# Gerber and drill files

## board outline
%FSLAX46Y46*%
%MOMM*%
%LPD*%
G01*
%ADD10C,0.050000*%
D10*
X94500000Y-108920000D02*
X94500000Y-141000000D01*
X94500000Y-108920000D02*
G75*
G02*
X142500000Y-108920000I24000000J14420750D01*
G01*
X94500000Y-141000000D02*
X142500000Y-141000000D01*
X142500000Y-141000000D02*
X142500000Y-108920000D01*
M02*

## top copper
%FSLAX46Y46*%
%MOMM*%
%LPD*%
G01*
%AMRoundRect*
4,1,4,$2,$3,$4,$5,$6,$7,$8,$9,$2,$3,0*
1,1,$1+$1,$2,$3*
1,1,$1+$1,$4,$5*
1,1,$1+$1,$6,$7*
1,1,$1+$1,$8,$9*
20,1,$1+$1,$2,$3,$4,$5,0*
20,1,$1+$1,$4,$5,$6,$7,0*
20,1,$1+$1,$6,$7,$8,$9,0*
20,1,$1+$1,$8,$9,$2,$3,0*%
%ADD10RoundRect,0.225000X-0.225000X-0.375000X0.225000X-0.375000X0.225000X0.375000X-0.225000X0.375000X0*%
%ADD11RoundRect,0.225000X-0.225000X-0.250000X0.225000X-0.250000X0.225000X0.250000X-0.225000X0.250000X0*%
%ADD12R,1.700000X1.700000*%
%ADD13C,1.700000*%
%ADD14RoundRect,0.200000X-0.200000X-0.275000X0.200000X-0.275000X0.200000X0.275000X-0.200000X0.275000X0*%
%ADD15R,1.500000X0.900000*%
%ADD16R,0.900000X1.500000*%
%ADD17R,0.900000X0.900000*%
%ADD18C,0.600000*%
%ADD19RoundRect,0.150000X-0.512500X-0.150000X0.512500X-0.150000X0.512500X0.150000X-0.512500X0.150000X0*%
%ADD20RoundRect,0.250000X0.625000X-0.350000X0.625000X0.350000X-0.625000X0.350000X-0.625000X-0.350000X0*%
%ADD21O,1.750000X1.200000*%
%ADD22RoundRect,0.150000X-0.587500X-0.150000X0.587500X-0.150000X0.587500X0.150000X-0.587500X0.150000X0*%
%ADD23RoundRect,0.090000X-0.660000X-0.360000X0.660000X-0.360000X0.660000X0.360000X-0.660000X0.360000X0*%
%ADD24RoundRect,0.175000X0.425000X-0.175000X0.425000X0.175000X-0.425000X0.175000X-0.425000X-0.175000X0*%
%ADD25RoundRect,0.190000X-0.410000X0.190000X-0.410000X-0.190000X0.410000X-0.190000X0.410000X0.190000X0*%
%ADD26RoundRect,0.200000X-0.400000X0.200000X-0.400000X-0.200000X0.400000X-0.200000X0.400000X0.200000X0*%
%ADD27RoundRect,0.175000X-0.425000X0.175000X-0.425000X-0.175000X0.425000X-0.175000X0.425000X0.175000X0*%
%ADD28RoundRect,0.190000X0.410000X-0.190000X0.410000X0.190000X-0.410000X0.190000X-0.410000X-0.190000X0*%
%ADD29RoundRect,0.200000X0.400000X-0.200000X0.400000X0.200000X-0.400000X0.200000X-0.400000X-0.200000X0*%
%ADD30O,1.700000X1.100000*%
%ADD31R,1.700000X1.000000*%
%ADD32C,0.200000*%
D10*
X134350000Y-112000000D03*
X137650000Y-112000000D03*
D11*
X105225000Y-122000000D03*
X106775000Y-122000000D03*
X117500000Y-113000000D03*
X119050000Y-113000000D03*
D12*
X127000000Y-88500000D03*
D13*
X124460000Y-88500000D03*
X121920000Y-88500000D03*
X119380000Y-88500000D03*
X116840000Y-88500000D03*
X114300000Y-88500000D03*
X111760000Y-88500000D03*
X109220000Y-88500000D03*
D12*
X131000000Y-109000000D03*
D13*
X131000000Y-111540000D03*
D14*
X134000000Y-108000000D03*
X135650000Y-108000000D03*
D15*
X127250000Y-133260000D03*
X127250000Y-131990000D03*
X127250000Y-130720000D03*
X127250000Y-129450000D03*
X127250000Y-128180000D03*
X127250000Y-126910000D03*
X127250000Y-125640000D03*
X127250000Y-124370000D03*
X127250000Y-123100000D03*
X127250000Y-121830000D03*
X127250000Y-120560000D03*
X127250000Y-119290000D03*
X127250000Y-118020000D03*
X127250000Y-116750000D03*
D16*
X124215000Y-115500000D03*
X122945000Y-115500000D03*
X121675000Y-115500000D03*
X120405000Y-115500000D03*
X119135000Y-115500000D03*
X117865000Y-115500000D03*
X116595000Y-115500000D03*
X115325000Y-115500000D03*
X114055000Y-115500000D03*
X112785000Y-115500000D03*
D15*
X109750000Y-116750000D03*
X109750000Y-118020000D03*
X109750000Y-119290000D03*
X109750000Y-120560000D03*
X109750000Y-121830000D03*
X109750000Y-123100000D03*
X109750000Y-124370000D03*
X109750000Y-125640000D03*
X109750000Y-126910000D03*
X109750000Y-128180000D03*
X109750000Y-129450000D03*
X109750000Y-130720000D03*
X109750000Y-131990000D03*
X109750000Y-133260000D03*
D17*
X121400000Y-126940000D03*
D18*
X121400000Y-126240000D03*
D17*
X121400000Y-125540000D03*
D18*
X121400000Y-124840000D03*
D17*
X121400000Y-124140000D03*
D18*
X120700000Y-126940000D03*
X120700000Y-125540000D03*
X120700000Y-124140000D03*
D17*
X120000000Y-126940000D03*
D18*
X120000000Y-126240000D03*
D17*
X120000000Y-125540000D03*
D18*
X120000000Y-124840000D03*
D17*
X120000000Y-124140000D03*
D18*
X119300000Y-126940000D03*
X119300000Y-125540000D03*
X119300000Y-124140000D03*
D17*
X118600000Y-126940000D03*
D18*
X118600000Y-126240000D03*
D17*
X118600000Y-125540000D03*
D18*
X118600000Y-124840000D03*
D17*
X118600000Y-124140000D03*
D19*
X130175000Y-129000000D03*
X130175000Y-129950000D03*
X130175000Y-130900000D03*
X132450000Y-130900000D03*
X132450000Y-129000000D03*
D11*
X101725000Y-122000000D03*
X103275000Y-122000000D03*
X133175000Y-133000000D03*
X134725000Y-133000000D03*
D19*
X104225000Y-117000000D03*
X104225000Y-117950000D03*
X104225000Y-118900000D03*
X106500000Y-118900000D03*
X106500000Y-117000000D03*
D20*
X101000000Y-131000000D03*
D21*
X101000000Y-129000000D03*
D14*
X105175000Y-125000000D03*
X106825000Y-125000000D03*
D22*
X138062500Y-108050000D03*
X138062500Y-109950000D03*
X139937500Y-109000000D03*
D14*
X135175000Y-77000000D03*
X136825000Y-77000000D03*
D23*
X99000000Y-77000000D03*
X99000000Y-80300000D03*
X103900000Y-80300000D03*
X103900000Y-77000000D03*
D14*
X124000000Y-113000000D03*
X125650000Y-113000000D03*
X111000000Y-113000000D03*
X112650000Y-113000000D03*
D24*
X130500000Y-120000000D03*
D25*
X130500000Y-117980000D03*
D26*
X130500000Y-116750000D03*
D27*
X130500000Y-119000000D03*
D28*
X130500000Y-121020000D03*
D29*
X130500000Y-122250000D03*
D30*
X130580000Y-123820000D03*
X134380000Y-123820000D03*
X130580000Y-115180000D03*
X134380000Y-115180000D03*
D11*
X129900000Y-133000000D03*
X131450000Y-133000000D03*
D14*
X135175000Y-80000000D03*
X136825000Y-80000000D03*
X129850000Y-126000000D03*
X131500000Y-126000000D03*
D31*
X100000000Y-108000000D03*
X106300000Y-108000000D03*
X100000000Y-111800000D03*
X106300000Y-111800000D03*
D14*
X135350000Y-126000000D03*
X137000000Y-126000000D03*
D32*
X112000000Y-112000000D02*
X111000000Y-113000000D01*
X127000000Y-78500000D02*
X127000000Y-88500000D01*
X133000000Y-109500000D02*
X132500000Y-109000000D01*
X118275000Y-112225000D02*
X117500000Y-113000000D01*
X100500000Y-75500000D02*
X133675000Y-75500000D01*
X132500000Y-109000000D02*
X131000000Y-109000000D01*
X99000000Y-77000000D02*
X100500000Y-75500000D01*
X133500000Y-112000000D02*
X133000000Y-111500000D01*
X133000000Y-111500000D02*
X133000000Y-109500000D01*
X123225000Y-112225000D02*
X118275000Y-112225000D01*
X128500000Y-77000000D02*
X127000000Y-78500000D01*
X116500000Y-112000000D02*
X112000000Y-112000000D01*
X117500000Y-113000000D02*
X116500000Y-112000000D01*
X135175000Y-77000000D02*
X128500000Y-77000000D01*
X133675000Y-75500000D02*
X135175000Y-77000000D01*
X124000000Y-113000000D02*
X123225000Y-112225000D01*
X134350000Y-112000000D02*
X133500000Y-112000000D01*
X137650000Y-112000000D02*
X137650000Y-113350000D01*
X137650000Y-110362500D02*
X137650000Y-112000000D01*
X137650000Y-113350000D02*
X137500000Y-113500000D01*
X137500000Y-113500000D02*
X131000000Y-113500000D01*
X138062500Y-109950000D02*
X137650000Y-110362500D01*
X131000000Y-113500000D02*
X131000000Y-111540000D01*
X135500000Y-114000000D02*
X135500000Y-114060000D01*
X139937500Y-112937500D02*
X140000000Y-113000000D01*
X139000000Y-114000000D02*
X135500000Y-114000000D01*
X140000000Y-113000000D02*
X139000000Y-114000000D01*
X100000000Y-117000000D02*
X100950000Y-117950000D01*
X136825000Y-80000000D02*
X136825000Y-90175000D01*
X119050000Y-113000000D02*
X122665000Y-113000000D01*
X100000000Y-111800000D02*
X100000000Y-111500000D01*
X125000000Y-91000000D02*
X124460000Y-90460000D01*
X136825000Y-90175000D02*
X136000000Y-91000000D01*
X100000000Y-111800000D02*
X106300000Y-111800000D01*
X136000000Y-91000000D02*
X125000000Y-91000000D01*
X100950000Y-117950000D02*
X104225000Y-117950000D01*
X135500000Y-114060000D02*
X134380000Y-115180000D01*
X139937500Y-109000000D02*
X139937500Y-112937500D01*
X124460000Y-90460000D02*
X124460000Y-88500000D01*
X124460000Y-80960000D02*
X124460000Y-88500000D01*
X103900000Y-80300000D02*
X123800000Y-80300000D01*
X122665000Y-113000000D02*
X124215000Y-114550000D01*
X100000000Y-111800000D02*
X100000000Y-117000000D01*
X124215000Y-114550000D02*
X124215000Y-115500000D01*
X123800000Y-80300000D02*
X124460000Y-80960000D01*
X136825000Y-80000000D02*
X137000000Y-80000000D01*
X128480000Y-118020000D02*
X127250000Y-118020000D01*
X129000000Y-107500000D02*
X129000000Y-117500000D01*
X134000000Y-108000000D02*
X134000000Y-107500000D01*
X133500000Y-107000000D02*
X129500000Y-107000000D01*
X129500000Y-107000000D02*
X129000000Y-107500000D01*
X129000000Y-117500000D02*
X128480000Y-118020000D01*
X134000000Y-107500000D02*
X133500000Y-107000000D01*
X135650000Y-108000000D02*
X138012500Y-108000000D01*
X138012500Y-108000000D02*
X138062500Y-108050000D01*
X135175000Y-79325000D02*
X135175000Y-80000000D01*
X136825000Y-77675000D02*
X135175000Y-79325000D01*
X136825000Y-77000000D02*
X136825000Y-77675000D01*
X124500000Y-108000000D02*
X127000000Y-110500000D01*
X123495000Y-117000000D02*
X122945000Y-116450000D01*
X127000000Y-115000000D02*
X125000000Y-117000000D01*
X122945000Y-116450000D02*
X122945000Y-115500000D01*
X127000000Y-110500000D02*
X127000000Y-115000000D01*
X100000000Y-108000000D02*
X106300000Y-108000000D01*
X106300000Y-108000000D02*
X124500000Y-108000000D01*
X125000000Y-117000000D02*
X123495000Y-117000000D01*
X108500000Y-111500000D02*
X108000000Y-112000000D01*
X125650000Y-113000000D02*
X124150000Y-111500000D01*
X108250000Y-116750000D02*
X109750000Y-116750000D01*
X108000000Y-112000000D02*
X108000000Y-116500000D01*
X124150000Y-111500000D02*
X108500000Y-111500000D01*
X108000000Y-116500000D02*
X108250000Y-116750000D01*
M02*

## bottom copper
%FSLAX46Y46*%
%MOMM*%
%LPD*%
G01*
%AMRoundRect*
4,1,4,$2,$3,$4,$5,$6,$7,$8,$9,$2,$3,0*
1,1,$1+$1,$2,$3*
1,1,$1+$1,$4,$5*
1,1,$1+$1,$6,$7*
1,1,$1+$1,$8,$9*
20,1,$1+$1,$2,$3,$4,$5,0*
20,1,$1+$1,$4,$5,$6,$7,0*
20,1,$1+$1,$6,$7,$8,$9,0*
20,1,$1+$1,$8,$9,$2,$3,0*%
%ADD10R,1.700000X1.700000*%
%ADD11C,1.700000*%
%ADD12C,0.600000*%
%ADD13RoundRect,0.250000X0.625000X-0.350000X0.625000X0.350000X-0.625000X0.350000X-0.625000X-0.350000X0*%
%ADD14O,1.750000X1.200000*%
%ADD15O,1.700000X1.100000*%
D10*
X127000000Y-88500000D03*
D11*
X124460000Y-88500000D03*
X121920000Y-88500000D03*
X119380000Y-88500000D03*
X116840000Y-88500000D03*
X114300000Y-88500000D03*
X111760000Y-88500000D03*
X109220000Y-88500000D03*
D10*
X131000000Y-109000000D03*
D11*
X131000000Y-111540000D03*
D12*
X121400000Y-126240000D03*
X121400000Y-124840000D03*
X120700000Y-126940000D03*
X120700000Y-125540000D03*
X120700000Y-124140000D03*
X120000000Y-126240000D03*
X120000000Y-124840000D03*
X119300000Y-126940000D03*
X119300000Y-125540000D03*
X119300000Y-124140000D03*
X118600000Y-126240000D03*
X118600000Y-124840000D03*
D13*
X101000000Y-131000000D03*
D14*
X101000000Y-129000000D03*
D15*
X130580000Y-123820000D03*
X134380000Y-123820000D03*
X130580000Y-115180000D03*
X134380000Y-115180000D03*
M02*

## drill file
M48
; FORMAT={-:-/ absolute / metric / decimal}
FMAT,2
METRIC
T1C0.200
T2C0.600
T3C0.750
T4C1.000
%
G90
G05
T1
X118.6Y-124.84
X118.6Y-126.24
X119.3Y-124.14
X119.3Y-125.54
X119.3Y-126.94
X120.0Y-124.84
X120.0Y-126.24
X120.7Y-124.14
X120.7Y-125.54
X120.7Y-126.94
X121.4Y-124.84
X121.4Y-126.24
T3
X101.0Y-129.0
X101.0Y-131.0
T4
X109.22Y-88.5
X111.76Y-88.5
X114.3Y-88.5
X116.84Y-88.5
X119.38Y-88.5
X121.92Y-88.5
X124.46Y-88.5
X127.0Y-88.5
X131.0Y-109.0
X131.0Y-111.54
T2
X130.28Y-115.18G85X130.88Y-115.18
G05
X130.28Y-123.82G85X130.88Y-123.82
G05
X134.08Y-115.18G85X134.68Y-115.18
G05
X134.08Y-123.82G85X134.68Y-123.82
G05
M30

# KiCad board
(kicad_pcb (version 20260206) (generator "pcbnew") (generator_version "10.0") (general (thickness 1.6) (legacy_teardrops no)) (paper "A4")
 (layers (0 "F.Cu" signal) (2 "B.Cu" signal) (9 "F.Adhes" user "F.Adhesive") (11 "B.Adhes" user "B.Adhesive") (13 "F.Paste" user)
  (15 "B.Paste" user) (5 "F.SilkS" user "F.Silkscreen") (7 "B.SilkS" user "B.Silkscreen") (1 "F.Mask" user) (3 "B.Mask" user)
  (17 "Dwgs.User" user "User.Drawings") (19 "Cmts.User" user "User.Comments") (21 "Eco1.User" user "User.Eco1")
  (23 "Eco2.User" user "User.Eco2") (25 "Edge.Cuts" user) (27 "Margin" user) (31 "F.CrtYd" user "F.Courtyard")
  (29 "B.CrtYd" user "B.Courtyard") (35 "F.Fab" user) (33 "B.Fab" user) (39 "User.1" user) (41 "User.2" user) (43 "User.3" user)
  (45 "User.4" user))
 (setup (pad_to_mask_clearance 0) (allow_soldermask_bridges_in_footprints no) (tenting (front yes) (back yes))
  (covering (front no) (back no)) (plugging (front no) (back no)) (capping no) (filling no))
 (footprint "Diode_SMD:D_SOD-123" (layer "F.Cu") (at 136 112)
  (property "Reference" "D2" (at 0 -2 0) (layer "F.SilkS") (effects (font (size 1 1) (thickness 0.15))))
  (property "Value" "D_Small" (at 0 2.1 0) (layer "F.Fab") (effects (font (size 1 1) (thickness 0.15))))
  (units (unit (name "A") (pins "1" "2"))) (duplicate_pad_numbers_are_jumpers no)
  (pad "1" smd roundrect (at -1.65 0) (size 0.9 1.2) (layers "F.Cu" "F.Mask" "F.Paste") (roundrect_rratio 0.25) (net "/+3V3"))
  (pad "2" smd roundrect (at 1.65 0) (size 0.9 1.2) (layers "F.Cu" "F.Mask" "F.Paste") (roundrect_rratio 0.25) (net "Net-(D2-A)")))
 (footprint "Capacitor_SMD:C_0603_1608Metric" (layer "F.Cu") (at 106 122)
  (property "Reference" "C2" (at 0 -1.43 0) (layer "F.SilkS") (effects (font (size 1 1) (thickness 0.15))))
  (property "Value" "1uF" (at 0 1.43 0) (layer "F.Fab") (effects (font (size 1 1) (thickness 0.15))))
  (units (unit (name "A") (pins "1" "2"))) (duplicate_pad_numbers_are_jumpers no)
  (pad "1" smd roundrect (at -0.775 0) (size 0.9 0.95) (layers "F.Cu" "F.Mask" "F.Paste") (roundrect_rratio 0.25) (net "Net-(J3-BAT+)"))
  (pad "2" smd roundrect (at 0.775 0) (size 0.9 0.95) (layers "F.Cu" "F.Mask" "F.Paste") (roundrect_rratio 0.25) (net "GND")))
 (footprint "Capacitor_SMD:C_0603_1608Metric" (layer "F.Cu") (at 118.275 113)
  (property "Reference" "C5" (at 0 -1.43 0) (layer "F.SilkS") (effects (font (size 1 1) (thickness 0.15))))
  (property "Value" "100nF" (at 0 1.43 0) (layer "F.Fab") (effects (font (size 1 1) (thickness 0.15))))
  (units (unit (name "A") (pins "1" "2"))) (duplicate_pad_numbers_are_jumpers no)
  (pad "1" smd roundrect (at -0.775 0) (size 0.9 0.95) (layers "F.Cu" "F.Mask" "F.Paste") (roundrect_rratio 0.25) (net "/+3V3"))
  (pad "2" smd roundrect (at 0.775 0) (size 0.9 0.95) (layers "F.Cu" "F.Mask" "F.Paste") (roundrect_rratio 0.25) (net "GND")))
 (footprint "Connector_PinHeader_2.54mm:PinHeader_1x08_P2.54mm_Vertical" (layer "F.Cu") (at 127 88.5 -90)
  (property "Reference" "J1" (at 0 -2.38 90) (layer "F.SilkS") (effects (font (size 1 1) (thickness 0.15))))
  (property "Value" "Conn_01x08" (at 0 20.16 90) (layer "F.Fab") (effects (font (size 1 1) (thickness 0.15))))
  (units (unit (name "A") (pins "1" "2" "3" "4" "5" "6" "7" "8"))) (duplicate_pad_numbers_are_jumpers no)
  (pad "1" thru_hole rect (at 0 0 270) (size 1.7 1.7) (drill 1) (layers "*.Cu" "*.Mask") (remove_unused_layers no) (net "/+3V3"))
  (pad "2" thru_hole circle (at 0 2.54 270) (size 1.7 1.7) (drill 1) (layers "*.Cu" "*.Mask") (remove_unused_layers no) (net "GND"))
  (pad "3" thru_hole circle (at 0 5.08 270) (size 1.7 1.7) (drill 1) (layers "*.Cu" "*.Mask") (remove_unused_layers no) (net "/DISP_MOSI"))
  (pad "4" thru_hole circle (at 0 7.62 270) (size 1.7 1.7) (drill 1) (layers "*.Cu" "*.Mask") (remove_unused_layers no) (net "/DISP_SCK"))
  (pad "5" thru_hole circle (at 0 10.16 270) (size 1.7 1.7) (drill 1) (layers "*.Cu" "*.Mask") (remove_unused_layers no) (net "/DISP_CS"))
  (pad "6" thru_hole circle (at 0 12.7 270) (size 1.7 1.7) (drill 1) (layers "*.Cu" "*.Mask") (remove_unused_layers no) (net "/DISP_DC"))
  (pad "7" thru_hole circle (at 0 15.24 270) (size 1.7 1.7) (drill 1) (layers "*.Cu" "*.Mask") (remove_unused_layers no) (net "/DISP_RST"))
  (pad "8" thru_hole circle (at 0 17.78 270) (size 1.7 1.7) (drill 1) (layers "*.Cu" "*.Mask") (remove_unused_layers no) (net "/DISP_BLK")))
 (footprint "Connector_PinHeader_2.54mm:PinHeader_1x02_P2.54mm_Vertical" (layer "F.Cu") (at 131 109)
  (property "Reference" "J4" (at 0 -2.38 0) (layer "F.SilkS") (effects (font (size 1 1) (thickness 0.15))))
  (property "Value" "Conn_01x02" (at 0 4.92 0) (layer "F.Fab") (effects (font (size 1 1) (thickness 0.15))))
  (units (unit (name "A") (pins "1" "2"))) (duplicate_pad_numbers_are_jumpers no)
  (pad "1" thru_hole rect (at 0 0) (size 1.7 1.7) (drill 1) (layers "*.Cu" "*.Mask") (remove_unused_layers no) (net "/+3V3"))
  (pad "2" thru_hole circle (at 0 2.54) (size 1.7 1.7) (drill 1) (layers "*.Cu" "*.Mask") (remove_unused_layers no) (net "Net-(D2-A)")))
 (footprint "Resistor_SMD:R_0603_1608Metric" (layer "F.Cu") (at 134.825 108)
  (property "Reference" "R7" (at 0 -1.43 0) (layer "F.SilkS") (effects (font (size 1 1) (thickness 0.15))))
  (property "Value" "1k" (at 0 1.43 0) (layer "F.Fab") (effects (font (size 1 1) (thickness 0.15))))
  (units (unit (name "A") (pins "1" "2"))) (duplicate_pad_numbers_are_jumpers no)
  (pad "1" smd roundrect (at -0.825 0) (size 0.8 0.95) (layers "F.Cu" "F.Mask" "F.Paste") (roundrect_rratio 0.25) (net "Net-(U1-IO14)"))
  (pad "2" smd roundrect (at 0.825 0) (size 0.8 0.95) (layers "F.Cu" "F.Mask" "F.Paste") (roundrect_rratio 0.25) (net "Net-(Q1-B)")))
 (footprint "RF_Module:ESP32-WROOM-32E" (layer "F.Cu") (at 118.5 128 180)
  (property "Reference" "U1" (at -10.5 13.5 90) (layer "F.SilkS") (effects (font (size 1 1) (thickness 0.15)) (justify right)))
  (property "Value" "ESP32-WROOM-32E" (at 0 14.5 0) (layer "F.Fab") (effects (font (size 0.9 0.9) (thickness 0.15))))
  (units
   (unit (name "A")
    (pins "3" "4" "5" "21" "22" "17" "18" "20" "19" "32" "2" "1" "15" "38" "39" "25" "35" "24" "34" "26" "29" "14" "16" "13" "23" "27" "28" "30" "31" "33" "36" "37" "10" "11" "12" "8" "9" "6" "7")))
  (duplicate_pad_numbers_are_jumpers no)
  (pad "1" smd rect (at -8.75 -5.26 180) (size 1.5 0.9) (layers "F.Cu" "F.Mask" "F.Paste") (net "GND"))
  (pad "2" smd rect (at -8.75 -3.99 180) (size 1.5 0.9) (layers "F.Cu" "F.Mask" "F.Paste") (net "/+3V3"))
  (pad "3" smd rect (at -8.75 -2.72 180) (size 1.5 0.9) (layers "F.Cu" "F.Mask" "F.Paste") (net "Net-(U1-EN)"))
  (pad "4" smd rect (at -8.75 -1.45 180) (size 1.5 0.9) (layers "F.Cu" "F.Mask" "F.Paste") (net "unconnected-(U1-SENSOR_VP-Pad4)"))
  (pad "5" smd rect (at -8.75 -0.18 180) (size 1.5 0.9) (layers "F.Cu" "F.Mask" "F.Paste") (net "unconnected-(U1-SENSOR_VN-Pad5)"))
  (pad "6" smd rect (at -8.75 1.09 180) (size 1.5 0.9) (layers "F.Cu" "F.Mask" "F.Paste") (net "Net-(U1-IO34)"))
  (pad "7" smd rect (at -8.75 2.36 180) (size 1.5 0.9) (layers "F.Cu" "F.Mask" "F.Paste") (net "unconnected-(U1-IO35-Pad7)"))
  (pad "8" smd rect (at -8.75 3.63 180) (size 1.5 0.9) (layers "F.Cu" "F.Mask" "F.Paste") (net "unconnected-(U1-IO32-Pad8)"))
  (pad "9" smd rect (at -8.75 4.9 180) (size 1.5 0.9) (layers "F.Cu" "F.Mask" "F.Paste") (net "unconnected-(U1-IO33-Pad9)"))
  (pad "10" smd rect (at -8.75 6.17 180) (size 1.5 0.9) (layers "F.Cu" "F.Mask" "F.Paste") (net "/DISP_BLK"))
  (pad "11" smd rect (at -8.75 7.44 180) (size 1.5 0.9) (layers "F.Cu" "F.Mask" "F.Paste") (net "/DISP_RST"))
  (pad "12" smd rect (at -8.75 8.71 180) (size 1.5 0.9) (layers "F.Cu" "F.Mask" "F.Paste") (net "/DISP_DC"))
  (pad "13" smd rect (at -8.75 9.98 180) (size 1.5 0.9) (layers "F.Cu" "F.Mask" "F.Paste") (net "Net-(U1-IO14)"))
  (pad "14" smd rect (at -8.75 11.25 180) (size 1.5 0.9) (layers "F.Cu" "F.Mask" "F.Paste") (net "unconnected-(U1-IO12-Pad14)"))
  (pad "15" smd rect (at -5.715 12.5 270) (size 1.5 0.9) (layers "F.Cu" "F.Mask" "F.Paste") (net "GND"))
  (pad "16" smd rect (at -4.445 12.5 270) (size 1.5 0.9) (layers "F.Cu" "F.Mask" "F.Paste") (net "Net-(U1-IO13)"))
  (pad "17" smd rect (at -3.175 12.5 270) (size 1.5 0.9) (layers "F.Cu" "F.Mask" "F.Paste") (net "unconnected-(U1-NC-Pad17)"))
  (pad "18" smd rect (at -1.905 12.5 270) (size 1.5 0.9) (layers "F.Cu" "F.Mask" "F.Paste") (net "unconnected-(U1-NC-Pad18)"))
  (pad "19" smd rect (at -0.635 12.5 270) (size 1.5 0.9) (layers "F.Cu" "F.Mask" "F.Paste") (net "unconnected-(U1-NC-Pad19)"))
  (pad "20" smd rect (at 0.635 12.5 270) (size 1.5 0.9) (layers "F.Cu" "F.Mask" "F.Paste") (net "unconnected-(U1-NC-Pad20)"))
  (pad "21" smd rect (at 1.905 12.5 270) (size 1.5 0.9) (layers "F.Cu" "F.Mask" "F.Paste") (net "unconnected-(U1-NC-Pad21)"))
  (pad "22" smd rect (at 3.175 12.5 270) (size 1.5 0.9) (layers "F.Cu" "F.Mask" "F.Paste") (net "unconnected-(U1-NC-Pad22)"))
  (pad "23" smd rect (at 4.445 12.5 270) (size 1.5 0.9) (layers "F.Cu" "F.Mask" "F.Paste") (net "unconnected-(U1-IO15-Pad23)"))
  (pad "24" smd rect (at 5.715 12.5 270) (size 1.5 0.9) (layers "F.Cu" "F.Mask" "F.Paste") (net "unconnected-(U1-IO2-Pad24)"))
  (pad "25" smd rect (at 8.75 11.25 180) (size 1.5 0.9) (layers "F.Cu" "F.Mask" "F.Paste") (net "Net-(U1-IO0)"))
  (pad "26" smd rect (at 8.75 9.98 180) (size 1.5 0.9) (layers "F.Cu" "F.Mask" "F.Paste") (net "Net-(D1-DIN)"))
  (pad "27" smd rect (at 8.75 8.71 180) (size 1.5 0.9) (layers "F.Cu" "F.Mask" "F.Paste") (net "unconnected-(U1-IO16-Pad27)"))
  (pad "28" smd rect (at 8.75 7.44 180) (size 1.5 0.9) (layers "F.Cu" "F.Mask" "F.Paste") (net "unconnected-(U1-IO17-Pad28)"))
  (pad "29" smd rect (at 8.75 6.17 180) (size 1.5 0.9) (layers "F.Cu" "F.Mask" "F.Paste") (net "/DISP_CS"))
  (pad "30" smd rect (at 8.75 4.9 180) (size 1.5 0.9) (layers "F.Cu" "F.Mask" "F.Paste") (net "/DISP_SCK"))
  (pad "31" smd rect (at 8.75 3.63 180) (size 1.5 0.9) (layers "F.Cu" "F.Mask" "F.Paste") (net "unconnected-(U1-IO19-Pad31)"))
  (pad "32" smd rect (at 8.75 2.36 180) (size 1.5 0.9) (layers "F.Cu" "F.Mask" "F.Paste") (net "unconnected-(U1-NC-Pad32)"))
  (pad "33" smd rect (at 8.75 1.09 180) (size 1.5 0.9) (layers "F.Cu" "F.Mask" "F.Paste") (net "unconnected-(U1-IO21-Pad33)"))
  (pad "34" smd rect (at 8.75 -0.18 180) (size 1.5 0.9) (layers "F.Cu" "F.Mask" "F.Paste") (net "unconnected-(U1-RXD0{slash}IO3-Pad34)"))
  (pad "35" smd rect (at 8.75 -1.45 180) (size 1.5 0.9) (layers "F.Cu" "F.Mask" "F.Paste") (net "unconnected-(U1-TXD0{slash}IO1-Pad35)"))
  (pad "36" smd rect (at 8.75 -2.72 180) (size 1.5 0.9) (layers "F.Cu" "F.Mask" "F.Paste") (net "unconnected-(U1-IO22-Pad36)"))
  (pad "37" smd rect (at 8.75 -3.99 180) (size 1.5 0.9) (layers "F.Cu" "F.Mask" "F.Paste") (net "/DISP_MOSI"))
  (pad "38" smd rect (at 8.75 -5.26 180) (size 1.5 0.9) (layers "F.Cu" "F.Mask" "F.Paste") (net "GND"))
  (pad "39" smd rect (at -2.9 1.06 180) (size 0.9 0.9) (layers "F.Cu" "F.Mask" "F.Paste") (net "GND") (zone_connect 2))
  (pad "39" thru_hole circle (at -2.9 1.76 180) (size 0.6 0.6) (drill 0.2) (layers "*.Cu" "*.Mask") (remove_unused_layers no) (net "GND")
   (zone_connect 2))
  (pad "39" smd rect (at -2.9 2.46 180) (size 0.9 0.9) (layers "F.Cu" "F.Mask" "F.Paste") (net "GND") (zone_connect 2))
  (pad "39" thru_hole circle (at -2.9 3.16 180) (size 0.6 0.6) (drill 0.2) (layers "*.Cu" "*.Mask") (remove_unused_layers no) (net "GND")
   (zone_connect 2))
  (pad "39" smd rect (at -2.9 3.86 180) (size 0.9 0.9) (layers "F.Cu" "F.Mask" "F.Paste") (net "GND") (zone_connect 2))
  (pad "39" thru_hole circle (at -2.2 1.06 180) (size 0.6 0.6) (drill 0.2) (layers "*.Cu" "*.Mask") (remove_unused_layers no) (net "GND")
   (zone_connect 2))
  (pad "39" thru_hole circle (at -2.2 2.46 180) (size 0.6 0.6) (drill 0.2) (layers "*.Cu" "*.Mask") (remove_unused_layers no) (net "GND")
   (zone_connect 2))
  (pad "39" thru_hole circle (at -2.2 3.86 180) (size 0.6 0.6) (drill 0.2) (layers "*.Cu" "*.Mask") (remove_unused_layers no) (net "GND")
   (zone_connect 2))
  (pad "39" smd rect (at -1.5 1.06 180) (size 0.9 0.9) (layers "F.Cu" "F.Mask" "F.Paste") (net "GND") (zone_connect 2))
  (pad "39" thru_hole circle (at -1.5 1.76 180) (size 0.6 0.6) (drill 0.2) (layers "*.Cu" "*.Mask") (remove_unused_layers no) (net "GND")
   (zone_connect 2))
  (pad "39" smd rect (at -1.5 2.46 180) (size 0.9 0.9) (layers "F.Cu" "F.Mask" "F.Paste") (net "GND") (zone_connect 2))
  (pad "39" thru_hole circle (at -1.5 3.16 180) (size 0.6 0.6) (drill 0.2) (layers "*.Cu" "*.Mask") (remove_unused_layers no) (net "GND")
   (zone_connect 2))
  (pad "39" smd rect (at -1.5 3.86 180) (size 0.9 0.9) (layers "F.Cu" "F.Mask" "F.Paste") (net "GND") (zone_connect 2))
  (pad "39" thru_hole circle (at -0.8 1.06 180) (size 0.6 0.6) (drill 0.2) (layers "*.Cu" "*.Mask") (remove_unused_layers no) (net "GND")
   (zone_connect 2))
  (pad "39" thru_hole circle (at -0.8 2.46 180) (size 0.6 0.6) (drill 0.2) (layers "*.Cu" "*.Mask") (remove_unused_layers no) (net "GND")
   (zone_connect 2))
  (pad "39" thru_hole circle (at -0.8 3.86 180) (size 0.6 0.6) (drill 0.2) (layers "*.Cu" "*.Mask") (remove_unused_layers no) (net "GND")
   (zone_connect 2))
  (pad "39" smd rect (at -0.1 1.06 180) (size 0.9 0.9) (layers "F.Cu" "F.Mask" "F.Paste") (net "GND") (zone_connect 2))
  (pad "39" thru_hole circle (at -0.1 1.76 180) (size 0.6 0.6) (drill 0.2) (layers "*.Cu" "*.Mask") (remove_unused_layers no) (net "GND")
   (zone_connect 2))
  (pad "39" smd rect (at -0.1 2.46 180) (size 0.9 0.9) (layers "F.Cu" "F.Mask" "F.Paste") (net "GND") (zone_connect 2))
  (pad "39" thru_hole circle (at -0.1 3.16 180) (size 0.6 0.6) (drill 0.2) (layers "*.Cu" "*.Mask") (remove_unused_layers no) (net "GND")
   (zone_connect 2))
  (pad "39" smd rect (at -0.1 3.86 180) (size 0.9 0.9) (layers "F.Cu" "F.Mask" "F.Paste") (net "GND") (zone_connect 2))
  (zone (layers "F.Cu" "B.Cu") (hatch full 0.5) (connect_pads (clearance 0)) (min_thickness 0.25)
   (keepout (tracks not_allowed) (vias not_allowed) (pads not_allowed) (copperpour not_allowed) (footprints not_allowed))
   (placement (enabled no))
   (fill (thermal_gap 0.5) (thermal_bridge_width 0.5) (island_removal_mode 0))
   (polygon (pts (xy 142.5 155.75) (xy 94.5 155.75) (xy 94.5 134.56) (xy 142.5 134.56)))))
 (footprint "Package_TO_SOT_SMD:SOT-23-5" (layer "F.Cu") (at 131.3125 129.95)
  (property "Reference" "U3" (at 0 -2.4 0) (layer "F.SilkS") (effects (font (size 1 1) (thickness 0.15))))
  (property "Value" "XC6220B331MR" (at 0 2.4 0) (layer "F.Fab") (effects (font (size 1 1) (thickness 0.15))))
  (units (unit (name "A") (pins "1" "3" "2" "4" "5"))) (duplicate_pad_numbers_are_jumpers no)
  (pad "1" smd roundrect (at -1.1375 -0.95) (size 1.325 0.6) (layers "F.Cu" "F.Mask" "F.Paste") (roundrect_rratio 0.25)
   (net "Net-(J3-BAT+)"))
  (pad "2" smd roundrect (at -1.1375 0) (size 1.325 0.6) (layers "F.Cu" "F.Mask" "F.Paste") (roundrect_rratio 0.25) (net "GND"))
  (pad "3" smd roundrect (at -1.1375 0.95) (size 1.325 0.6) (layers "F.Cu" "F.Mask" "F.Paste") (roundrect_rratio 0.25) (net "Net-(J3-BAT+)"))
  (pad "4" smd roundrect (at 1.1375 0.95) (size 1.325 0.6) (layers "F.Cu" "F.Mask" "F.Paste") (roundrect_rratio 0.25)
   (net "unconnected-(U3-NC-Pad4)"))
  (pad "5" smd roundrect (at 1.1375 -0.95) (size 1.325 0.6) (layers "F.Cu" "F.Mask" "F.Paste") (roundrect_rratio 0.25) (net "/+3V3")))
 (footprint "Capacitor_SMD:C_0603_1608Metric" (layer "F.Cu") (at 102.5 122)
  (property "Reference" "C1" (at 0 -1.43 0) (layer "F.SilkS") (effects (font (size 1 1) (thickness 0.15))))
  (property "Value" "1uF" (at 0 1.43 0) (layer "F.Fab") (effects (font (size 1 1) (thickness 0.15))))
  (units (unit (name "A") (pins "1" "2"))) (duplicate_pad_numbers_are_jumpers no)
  (pad "1" smd roundrect (at -0.775 0) (size 0.9 0.95) (layers "F.Cu" "F.Mask" "F.Paste") (roundrect_rratio 0.25) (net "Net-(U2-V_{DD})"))
  (pad "2" smd roundrect (at 0.775 0) (size 0.9 0.95) (layers "F.Cu" "F.Mask" "F.Paste") (roundrect_rratio 0.25) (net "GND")))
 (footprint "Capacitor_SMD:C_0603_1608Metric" (layer "F.Cu") (at 133.95 133)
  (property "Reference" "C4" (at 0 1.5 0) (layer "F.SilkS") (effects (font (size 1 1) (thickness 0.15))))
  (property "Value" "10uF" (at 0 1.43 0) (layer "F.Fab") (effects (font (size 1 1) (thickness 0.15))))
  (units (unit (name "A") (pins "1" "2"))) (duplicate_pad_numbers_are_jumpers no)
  (pad "1" smd roundrect (at -0.775 0) (size 0.9 0.95) (layers "F.Cu" "F.Mask" "F.Paste") (roundrect_rratio 0.25) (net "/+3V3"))
  (pad "2" smd roundrect (at 0.775 0) (size 0.9 0.95) (layers "F.Cu" "F.Mask" "F.Paste") (roundrect_rratio 0.25) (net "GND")))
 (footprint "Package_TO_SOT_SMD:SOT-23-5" (layer "F.Cu") (at 105.3625 117.95)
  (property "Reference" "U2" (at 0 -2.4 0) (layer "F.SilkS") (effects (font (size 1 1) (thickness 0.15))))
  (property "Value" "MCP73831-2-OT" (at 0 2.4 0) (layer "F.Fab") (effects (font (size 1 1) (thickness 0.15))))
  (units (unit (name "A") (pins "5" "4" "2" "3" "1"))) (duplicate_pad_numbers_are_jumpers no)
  (pad "1" smd roundrect (at -1.1375 -0.95) (size 1.325 0.6) (layers "F.Cu" "F.Mask" "F.Paste") (roundrect_rratio 0.25)
   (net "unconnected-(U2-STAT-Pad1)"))
  (pad "2" smd roundrect (at -1.1375 0) (size 1.325 0.6) (layers "F.Cu" "F.Mask" "F.Paste") (roundrect_rratio 0.25) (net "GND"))
  (pad "3" smd roundrect (at -1.1375 0.95) (size 1.325 0.6) (layers "F.Cu" "F.Mask" "F.Paste") (roundrect_rratio 0.25) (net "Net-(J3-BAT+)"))
  (pad "4" smd roundrect (at 1.1375 0.95) (size 1.325 0.6) (layers "F.Cu" "F.Mask" "F.Paste") (roundrect_rratio 0.25)
   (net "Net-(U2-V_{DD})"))
  (pad "5" smd roundrect (at 1.1375 -0.95) (size 1.325 0.6) (layers "F.Cu" "F.Mask" "F.Paste") (roundrect_rratio 0.25) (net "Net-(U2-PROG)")))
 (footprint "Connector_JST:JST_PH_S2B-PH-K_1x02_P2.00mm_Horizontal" (layer "F.Cu") (at 101 131 90)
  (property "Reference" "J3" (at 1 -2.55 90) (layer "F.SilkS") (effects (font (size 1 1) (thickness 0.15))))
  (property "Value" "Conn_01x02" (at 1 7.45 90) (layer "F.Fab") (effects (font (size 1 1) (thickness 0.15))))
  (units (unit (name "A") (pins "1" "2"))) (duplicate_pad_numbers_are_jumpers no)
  (pad "1" thru_hole roundrect (at 0 0 90) (size 1.2 1.75) (drill 0.75) (layers "*.Cu" "*.Mask") (remove_unused_layers no)
   (roundrect_rratio 0.208333) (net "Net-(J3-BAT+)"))
  (pad "2" thru_hole oval (at 2 0 90) (size 1.2 1.75) (drill 0.75) (layers "*.Cu" "*.Mask") (remove_unused_layers no) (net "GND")))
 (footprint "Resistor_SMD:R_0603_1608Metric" (layer "F.Cu") (at 106 125)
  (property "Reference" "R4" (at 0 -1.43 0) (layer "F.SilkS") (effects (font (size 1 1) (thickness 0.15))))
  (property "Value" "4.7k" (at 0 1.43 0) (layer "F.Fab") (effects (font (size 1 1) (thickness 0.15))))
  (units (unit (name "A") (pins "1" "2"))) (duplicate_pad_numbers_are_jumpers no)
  (pad "1" smd roundrect (at -0.825 0) (size 0.8 0.95) (layers "F.Cu" "F.Mask" "F.Paste") (roundrect_rratio 0.25) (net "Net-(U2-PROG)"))
  (pad "2" smd roundrect (at 0.825 0) (size 0.8 0.95) (layers "F.Cu" "F.Mask" "F.Paste") (roundrect_rratio 0.25) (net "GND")))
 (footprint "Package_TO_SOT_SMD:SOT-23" (layer "F.Cu") (at 139 109)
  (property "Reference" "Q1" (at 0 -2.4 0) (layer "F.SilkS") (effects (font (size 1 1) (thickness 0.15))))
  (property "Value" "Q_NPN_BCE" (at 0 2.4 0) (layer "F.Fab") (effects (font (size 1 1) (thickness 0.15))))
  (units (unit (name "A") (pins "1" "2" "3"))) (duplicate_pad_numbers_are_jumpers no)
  (pad "1" smd roundrect (at -0.9375 -0.95) (size 1.475 0.6) (layers "F.Cu" "F.Mask" "F.Paste") (roundrect_rratio 0.25) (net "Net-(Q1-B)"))
  (pad "2" smd roundrect (at -0.9375 0.95) (size 1.475 0.6) (layers "F.Cu" "F.Mask" "F.Paste") (roundrect_rratio 0.25) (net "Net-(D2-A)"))
  (pad "3" smd roundrect (at 0.9375 0) (size 1.475 0.6) (layers "F.Cu" "F.Mask" "F.Paste") (roundrect_rratio 0.25) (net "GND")))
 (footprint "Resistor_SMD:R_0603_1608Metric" (layer "F.Cu") (at 136 77)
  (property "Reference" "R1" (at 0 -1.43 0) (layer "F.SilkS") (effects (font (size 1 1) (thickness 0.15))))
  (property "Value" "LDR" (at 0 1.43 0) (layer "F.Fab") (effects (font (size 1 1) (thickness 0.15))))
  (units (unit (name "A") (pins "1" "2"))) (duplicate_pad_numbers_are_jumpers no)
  (pad "1" smd roundrect (at -0.825 0) (size 0.8 0.95) (layers "F.Cu" "F.Mask" "F.Paste") (roundrect_rratio 0.25) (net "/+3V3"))
  (pad "2" smd roundrect (at 0.825 0) (size 0.8 0.95) (layers "F.Cu" "F.Mask" "F.Paste") (roundrect_rratio 0.25) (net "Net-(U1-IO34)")))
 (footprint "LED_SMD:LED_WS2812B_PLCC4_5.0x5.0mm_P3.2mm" (layer "F.Cu") (at 101.45 78.65)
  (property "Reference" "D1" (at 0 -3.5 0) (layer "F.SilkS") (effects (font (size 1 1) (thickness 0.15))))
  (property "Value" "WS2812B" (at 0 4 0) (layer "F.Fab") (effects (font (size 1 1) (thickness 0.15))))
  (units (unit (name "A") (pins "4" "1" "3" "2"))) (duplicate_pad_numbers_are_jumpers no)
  (pad "1" smd roundrect (at -2.45 -1.65) (size 1.5 0.9) (layers "F.Cu" "F.Mask" "F.Paste") (roundrect_rratio 0.1) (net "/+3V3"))
  (pad "2" smd roundrect (at -2.45 1.65) (size 1.5 0.9) (layers "F.Cu" "F.Mask" "F.Paste") (roundrect_rratio 0.1)
   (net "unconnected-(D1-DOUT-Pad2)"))
  (pad "3" smd roundrect (at 2.45 1.65) (size 1.5 0.9) (layers "F.Cu" "F.Mask" "F.Paste") (roundrect_rratio 0.1) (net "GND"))
  (pad "4" smd roundrect (at 2.45 -1.65) (size 1.5 0.9) (layers "F.Cu" "F.Mask" "F.Paste") (roundrect_rratio 0.1) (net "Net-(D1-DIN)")))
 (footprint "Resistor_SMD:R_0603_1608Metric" (layer "F.Cu") (at 124.825 113)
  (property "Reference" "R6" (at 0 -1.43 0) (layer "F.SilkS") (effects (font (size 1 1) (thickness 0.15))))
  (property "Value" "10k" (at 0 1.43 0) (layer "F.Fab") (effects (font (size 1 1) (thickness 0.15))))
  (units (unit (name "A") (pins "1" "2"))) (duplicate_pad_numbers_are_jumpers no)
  (pad "1" smd roundrect (at -0.825 0) (size 0.8 0.95) (layers "F.Cu" "F.Mask" "F.Paste") (roundrect_rratio 0.25) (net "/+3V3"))
  (pad "2" smd roundrect (at 0.825 0) (size 0.8 0.95) (layers "F.Cu" "F.Mask" "F.Paste") (roundrect_rratio 0.25) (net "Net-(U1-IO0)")))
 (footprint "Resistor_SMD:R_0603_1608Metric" (layer "F.Cu") (at 111.825 113)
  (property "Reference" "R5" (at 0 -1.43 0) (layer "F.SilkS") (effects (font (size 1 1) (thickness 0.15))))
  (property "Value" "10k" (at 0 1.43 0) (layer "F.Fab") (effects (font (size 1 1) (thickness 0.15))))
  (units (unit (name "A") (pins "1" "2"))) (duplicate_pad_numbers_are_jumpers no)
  (pad "1" smd roundrect (at -0.825 0) (size 0.8 0.95) (layers "F.Cu" "F.Mask" "F.Paste") (roundrect_rratio 0.25) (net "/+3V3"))
  (pad "2" smd roundrect (at 0.825 0) (size 0.8 0.95) (layers "F.Cu" "F.Mask" "F.Paste") (roundrect_rratio 0.25) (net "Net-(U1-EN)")))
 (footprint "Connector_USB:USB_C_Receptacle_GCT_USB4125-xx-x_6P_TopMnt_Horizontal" (layer "F.Cu") (at 133.58 119.5 90)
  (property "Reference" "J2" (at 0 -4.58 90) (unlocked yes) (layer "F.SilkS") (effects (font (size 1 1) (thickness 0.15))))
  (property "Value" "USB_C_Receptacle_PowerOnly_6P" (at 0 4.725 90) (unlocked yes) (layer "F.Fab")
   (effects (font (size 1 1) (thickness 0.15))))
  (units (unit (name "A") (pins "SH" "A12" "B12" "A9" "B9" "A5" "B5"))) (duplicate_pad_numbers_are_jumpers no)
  (pad "A5" smd roundrect (at -0.5 -3.08 90) (size 0.7 1.2) (layers "F.Cu" "F.Mask" "F.Paste") (roundrect_rratio 0.25) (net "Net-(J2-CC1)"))
  (pad "A9" smd roundrect (at 1.52 -3.08 270) (size 0.76 1.2) (layers "F.Cu" "F.Mask" "F.Paste") (roundrect_rratio 0.25)
   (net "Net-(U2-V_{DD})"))
  (pad "A12" smd roundrect (at 2.75 -3.08 270) (size 0.8 1.2) (layers "F.Cu" "F.Mask" "F.Paste") (roundrect_rratio 0.25) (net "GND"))
  (pad "B5" smd roundrect (at 0.5 -3.08 270) (size 0.7 1.2) (layers "F.Cu" "F.Mask" "F.Paste") (roundrect_rratio 0.25) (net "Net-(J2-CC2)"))
  (pad "B9" smd roundrect (at -1.52 -3.08 90) (size 0.76 1.2) (layers "F.Cu" "F.Mask" "F.Paste") (roundrect_rratio 0.25)
   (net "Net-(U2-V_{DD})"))
  (pad "B12" smd roundrect (at -2.75 -3.08 90) (size 0.8 1.2) (layers "F.Cu" "F.Mask" "F.Paste") (roundrect_rratio 0.25) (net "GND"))
  (pad "SH" thru_hole oval (at -4.32 -3 90) (size 1.1 1.7) (drill oval 0.6 1.2) (layers "*.Cu" "*.Mask" "F.Paste") (remove_unused_layers no)
   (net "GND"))
  (pad "SH" thru_hole oval (at -4.32 0.8 90) (size 1.1 1.7) (drill oval 0.6 1.2) (layers "*.Cu" "*.Mask" "F.Paste")
   (remove_unused_layers no) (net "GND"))
  (pad "SH" thru_hole oval (at 4.32 -3 90) (size 1.1 1.7) (drill oval 0.6 1.2) (layers "*.Cu" "*.Mask" "F.Paste") (remove_unused_layers no)
   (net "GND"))
  (pad "SH" thru_hole oval (at 4.32 0.8 90) (size 1.1 1.7) (drill oval 0.6 1.2) (layers "*.Cu" "*.Mask" "F.Paste") (remove_unused_layers no)
   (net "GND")))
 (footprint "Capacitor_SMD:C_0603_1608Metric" (layer "F.Cu") (at 130.675 133)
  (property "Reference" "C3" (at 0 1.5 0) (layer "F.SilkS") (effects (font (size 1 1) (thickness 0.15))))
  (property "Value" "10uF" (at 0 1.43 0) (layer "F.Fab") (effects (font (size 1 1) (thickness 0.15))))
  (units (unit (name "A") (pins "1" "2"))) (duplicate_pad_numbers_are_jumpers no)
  (pad "1" smd roundrect (at -0.775 0) (size 0.9 0.95) (layers "F.Cu" "F.Mask" "F.Paste") (roundrect_rratio 0.25) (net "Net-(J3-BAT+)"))
  (pad "2" smd roundrect (at 0.775 0) (size 0.9 0.95) (layers "F.Cu" "F.Mask" "F.Paste") (roundrect_rratio 0.25) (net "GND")))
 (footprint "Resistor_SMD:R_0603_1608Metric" (layer "F.Cu") (at 136 80)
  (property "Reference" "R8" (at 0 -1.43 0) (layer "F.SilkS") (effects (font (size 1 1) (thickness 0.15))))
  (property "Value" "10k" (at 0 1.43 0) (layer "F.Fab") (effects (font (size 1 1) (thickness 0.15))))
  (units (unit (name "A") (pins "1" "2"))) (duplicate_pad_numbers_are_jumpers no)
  (pad "1" smd roundrect (at -0.825 0) (size 0.8 0.95) (layers "F.Cu" "F.Mask" "F.Paste") (roundrect_rratio 0.25) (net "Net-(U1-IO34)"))
  (pad "2" smd roundrect (at 0.825 0) (size 0.8 0.95) (layers "F.Cu" "F.Mask" "F.Paste") (roundrect_rratio 0.25) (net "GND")))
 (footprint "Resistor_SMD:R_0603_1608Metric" (layer "F.Cu") (at 130.675 126)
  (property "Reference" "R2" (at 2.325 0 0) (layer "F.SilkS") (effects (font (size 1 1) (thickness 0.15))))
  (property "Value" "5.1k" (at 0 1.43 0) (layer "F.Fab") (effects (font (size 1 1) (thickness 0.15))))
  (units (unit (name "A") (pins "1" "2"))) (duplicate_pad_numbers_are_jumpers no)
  (pad "1" smd roundrect (at -0.825 0) (size 0.8 0.95) (layers "F.Cu" "F.Mask" "F.Paste") (roundrect_rratio 0.25) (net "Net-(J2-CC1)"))
  (pad "2" smd roundrect (at 0.825 0) (size 0.8 0.95) (layers "F.Cu" "F.Mask" "F.Paste") (roundrect_rratio 0.25) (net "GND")))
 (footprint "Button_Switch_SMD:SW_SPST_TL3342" (layer "F.Cu") (at 103.15 109.9)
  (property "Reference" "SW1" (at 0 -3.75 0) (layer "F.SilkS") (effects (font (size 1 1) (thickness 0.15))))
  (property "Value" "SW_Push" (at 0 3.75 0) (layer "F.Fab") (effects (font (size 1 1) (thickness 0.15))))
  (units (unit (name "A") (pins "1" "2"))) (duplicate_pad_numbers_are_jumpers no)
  (pad "1" smd rect (at -3.15 -1.9) (size 1.7 1) (layers "F.Cu" "F.Mask" "F.Paste") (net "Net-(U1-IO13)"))
  (pad "1" smd rect (at 3.15 -1.9) (size 1.7 1) (layers "F.Cu" "F.Mask" "F.Paste") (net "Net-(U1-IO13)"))
  (pad "2" smd rect (at -3.15 1.9) (size 1.7 1) (layers "F.Cu" "F.Mask" "F.Paste") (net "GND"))
  (pad "2" smd rect (at 3.15 1.9) (size 1.7 1) (layers "F.Cu" "F.Mask" "F.Paste") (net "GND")))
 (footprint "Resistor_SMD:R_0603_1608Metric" (layer "F.Cu") (at 136.175 126)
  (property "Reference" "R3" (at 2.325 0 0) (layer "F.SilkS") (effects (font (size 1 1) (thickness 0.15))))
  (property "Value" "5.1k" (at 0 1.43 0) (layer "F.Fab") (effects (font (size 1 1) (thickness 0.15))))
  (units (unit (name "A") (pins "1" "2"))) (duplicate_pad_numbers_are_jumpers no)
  (pad "1" smd roundrect (at -0.825 0) (size 0.8 0.95) (layers "F.Cu" "F.Mask" "F.Paste") (roundrect_rratio 0.25) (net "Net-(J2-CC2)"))
  (pad "2" smd roundrect (at 0.825 0) (size 0.8 0.95) (layers "F.Cu" "F.Mask" "F.Paste") (roundrect_rratio 0.25) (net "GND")))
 (gr_line (start 94.5 108.92) (end 94.5 141) (stroke (width 0.05) (type solid)) (layer "Edge.Cuts"))
 (gr_arc (start 94.5 108.92) (mid 118.5 66.5) (end 142.5 108.92) (stroke (width 0.05) (type solid)) (layer "Edge.Cuts"))
 (gr_line (start 94.5 141) (end 142.5 141) (stroke (width 0.05) (type solid)) (layer "Edge.Cuts"))
 (gr_line (start 142.5 141) (end 142.5 108.92) (stroke (width 0.05) (type solid)) (layer "Edge.Cuts"))
 (segment (start 112 112) (end 111 113) (width 0.2) (layer "F.Cu") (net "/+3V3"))
 (segment (start 127 78.5) (end 127 88.5) (width 0.2) (layer "F.Cu") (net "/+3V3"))
 (segment (start 133 109.5) (end 132.5 109) (width 0.2) (layer "F.Cu") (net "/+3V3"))
 (segment (start 118.275 112.225) (end 117.5 113) (width 0.2) (layer "F.Cu") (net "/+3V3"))
 (segment (start 100.5 75.5) (end 133.675 75.5) (width 0.2) (layer "F.Cu") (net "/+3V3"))
 (segment (start 132.5 109) (end 131 109) (width 0.2) (layer "F.Cu") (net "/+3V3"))
 (segment (start 99 77) (end 100.5 75.5) (width 0.2) (layer "F.Cu") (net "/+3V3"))
 (segment (start 133.5 112) (end 133 111.5) (width 0.2) (layer "F.Cu") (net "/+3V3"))
 (segment (start 133 111.5) (end 133 109.5) (width 0.2) (layer "F.Cu") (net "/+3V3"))
 (segment (start 123.225 112.225) (end 118.275 112.225) (width 0.2) (layer "F.Cu") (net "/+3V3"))
 (segment (start 128.5 77) (end 127 78.5) (width 0.2) (layer "F.Cu") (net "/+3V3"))
 (segment (start 116.5 112) (end 112 112) (width 0.2) (layer "F.Cu") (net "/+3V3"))
 (segment (start 117.5 113) (end 116.5 112) (width 0.2) (layer "F.Cu") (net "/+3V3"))
 (segment (start 135.175 77) (end 128.5 77) (width 0.2) (layer "F.Cu") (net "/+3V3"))
 (segment (start 133.675 75.5) (end 135.175 77) (width 0.2) (layer "F.Cu") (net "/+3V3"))
 (segment (start 124 113) (end 123.225 112.225) (width 0.2) (layer "F.Cu") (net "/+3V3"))
 (segment (start 134.35 112) (end 133.5 112) (width 0.2) (layer "F.Cu") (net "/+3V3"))
 (segment (start 137.65 112) (end 137.65 113.35) (width 0.2) (layer "F.Cu") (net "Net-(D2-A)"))
 (segment (start 137.65 110.3625) (end 137.65 112) (width 0.2) (layer "F.Cu") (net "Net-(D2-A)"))
 (segment (start 137.65 113.35) (end 137.5 113.5) (width 0.2) (layer "F.Cu") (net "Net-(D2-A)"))
 (segment (start 137.5 113.5) (end 131 113.5) (width 0.2) (layer "F.Cu") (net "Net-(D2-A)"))
 (segment (start 138.0625 109.95) (end 137.65 110.3625) (width 0.2) (layer "F.Cu") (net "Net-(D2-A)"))
 (segment (start 131 113.5) (end 131 111.54) (width 0.2) (layer "F.Cu") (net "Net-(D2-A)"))
 (segment (start 135.5 114) (end 135.5 114.06) (width 0.2) (layer "F.Cu") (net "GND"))
 (segment (start 139.9375 112.9375) (end 140 113) (width 0.2) (layer "F.Cu") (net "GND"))
 (segment (start 139 114) (end 135.5 114) (width 0.2) (layer "F.Cu") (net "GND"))
 (segment (start 140 113) (end 139 114) (width 0.2) (layer "F.Cu") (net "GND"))
 (segment (start 100 117) (end 100.95 117.95) (width 0.2) (layer "F.Cu") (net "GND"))
 (segment (start 136.825 80) (end 136.825 90.175) (width 0.2) (layer "F.Cu") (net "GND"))
 (segment (start 119.05 113) (end 122.665 113) (width 0.2) (layer "F.Cu") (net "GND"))
 (segment (start 100 111.8) (end 100 111.5) (width 0.2) (layer "F.Cu") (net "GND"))
 (segment (start 125 91) (end 124.46 90.46) (width 0.2) (layer "F.Cu") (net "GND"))
 (segment (start 136.825 90.175) (end 136 91) (width 0.2) (layer "F.Cu") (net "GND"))
 (segment (start 100 111.8) (end 106.3 111.8) (width 0.2) (layer "F.Cu") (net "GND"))
 (segment (start 136 91) (end 125 91) (width 0.2) (layer "F.Cu") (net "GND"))
 (segment (start 100.95 117.95) (end 104.225 117.95) (width 0.2) (layer "F.Cu") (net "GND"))
 (segment (start 135.5 114.06) (end 134.38 115.18) (width 0.2) (layer "F.Cu") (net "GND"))
 (segment (start 139.9375 109) (end 139.9375 112.9375) (width 0.2) (layer "F.Cu") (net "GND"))
 (segment (start 124.46 90.46) (end 124.46 88.5) (width 0.2) (layer "F.Cu") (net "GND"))
 (segment (start 124.46 80.96) (end 124.46 88.5) (width 0.2) (layer "F.Cu") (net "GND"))
 (segment (start 103.9 80.3) (end 123.8 80.3) (width 0.2) (layer "F.Cu") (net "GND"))
 (segment (start 122.665 113) (end 124.215 114.55) (width 0.2) (layer "F.Cu") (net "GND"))
 (segment (start 100 111.8) (end 100 117) (width 0.2) (layer "F.Cu") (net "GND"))
 (segment (start 124.215 114.55) (end 124.215 115.5) (width 0.2) (layer "F.Cu") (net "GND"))
 (segment (start 123.8 80.3) (end 124.46 80.96) (width 0.2) (layer "F.Cu") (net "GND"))
 (segment (start 136.825 80) (end 137 80) (width 0.2) (layer "F.Cu") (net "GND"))
 (segment (start 128.48 118.02) (end 127.25 118.02) (width 0.2) (layer "F.Cu") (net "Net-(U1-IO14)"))
 (segment (start 129 107.5) (end 129 117.5) (width 0.2) (layer "F.Cu") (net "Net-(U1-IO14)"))
 (segment (start 134 108) (end 134 107.5) (width 0.2) (layer "F.Cu") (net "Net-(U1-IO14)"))
 (segment (start 133.5 107) (end 129.5 107) (width 0.2) (layer "F.Cu") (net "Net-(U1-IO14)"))
 (segment (start 129.5 107) (end 129 107.5) (width 0.2) (layer "F.Cu") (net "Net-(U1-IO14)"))
 (segment (start 129 117.5) (end 128.48 118.02) (width 0.2) (layer "F.Cu") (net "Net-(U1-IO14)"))
 (segment (start 134 107.5) (end 133.5 107) (width 0.2) (layer "F.Cu") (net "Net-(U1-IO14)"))
 (segment (start 135.65 108) (end 138.0125 108) (width 0.2) (layer "F.Cu") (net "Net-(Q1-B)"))
 (segment (start 138.0125 108) (end 138.0625 108.05) (width 0.2) (layer "F.Cu") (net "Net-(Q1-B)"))
 (segment (start 135.175 79.325) (end 135.175 80) (width 0.2) (layer "F.Cu") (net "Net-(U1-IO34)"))
 (segment (start 136.825 77.675) (end 135.175 79.325) (width 0.2) (layer "F.Cu") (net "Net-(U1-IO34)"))
 (segment (start 136.825 77) (end 136.825 77.675) (width 0.2) (layer "F.Cu") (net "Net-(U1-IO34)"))
 (segment (start 124.5 108) (end 127 110.5) (width 0.2) (layer "F.Cu") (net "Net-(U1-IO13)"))
 (segment (start 123.495 117) (end 122.945 116.45) (width 0.2) (layer "F.Cu") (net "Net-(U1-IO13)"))
 (segment (start 127 115) (end 125 117) (width 0.2) (layer "F.Cu") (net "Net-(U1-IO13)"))
 (segment (start 122.945 116.45) (end 122.945 115.5) (width 0.2) (layer "F.Cu") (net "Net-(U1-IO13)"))
 (segment (start 127 110.5) (end 127 115) (width 0.2) (layer "F.Cu") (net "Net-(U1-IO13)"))
 (segment (start 100 108) (end 106.3 108) (width 0.2) (layer "F.Cu") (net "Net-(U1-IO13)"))
 (segment (start 106.3 108) (end 124.5 108) (width 0.2) (layer "F.Cu") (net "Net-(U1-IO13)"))
 (segment (start 125 117) (end 123.495 117) (width 0.2) (layer "F.Cu") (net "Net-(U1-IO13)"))
 (segment (start 108.5 111.5) (end 108 112) (width 0.2) (layer "F.Cu") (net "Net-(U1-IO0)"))
 (segment (start 125.65 113) (end 124.15 111.5) (width 0.2) (layer "F.Cu") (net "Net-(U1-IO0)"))
 (segment (start 108.25 116.75) (end 109.75 116.75) (width 0.2) (layer "F.Cu") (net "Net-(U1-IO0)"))
 (segment (start 108 112) (end 108 116.5) (width 0.2) (layer "F.Cu") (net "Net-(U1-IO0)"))
 (segment (start 124.15 111.5) (end 108.5 111.5) (width 0.2) (layer "F.Cu") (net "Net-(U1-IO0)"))
 (segment (start 108 116.5) (end 108.25 116.75) (width 0.2) (layer "F.Cu") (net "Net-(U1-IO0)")))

